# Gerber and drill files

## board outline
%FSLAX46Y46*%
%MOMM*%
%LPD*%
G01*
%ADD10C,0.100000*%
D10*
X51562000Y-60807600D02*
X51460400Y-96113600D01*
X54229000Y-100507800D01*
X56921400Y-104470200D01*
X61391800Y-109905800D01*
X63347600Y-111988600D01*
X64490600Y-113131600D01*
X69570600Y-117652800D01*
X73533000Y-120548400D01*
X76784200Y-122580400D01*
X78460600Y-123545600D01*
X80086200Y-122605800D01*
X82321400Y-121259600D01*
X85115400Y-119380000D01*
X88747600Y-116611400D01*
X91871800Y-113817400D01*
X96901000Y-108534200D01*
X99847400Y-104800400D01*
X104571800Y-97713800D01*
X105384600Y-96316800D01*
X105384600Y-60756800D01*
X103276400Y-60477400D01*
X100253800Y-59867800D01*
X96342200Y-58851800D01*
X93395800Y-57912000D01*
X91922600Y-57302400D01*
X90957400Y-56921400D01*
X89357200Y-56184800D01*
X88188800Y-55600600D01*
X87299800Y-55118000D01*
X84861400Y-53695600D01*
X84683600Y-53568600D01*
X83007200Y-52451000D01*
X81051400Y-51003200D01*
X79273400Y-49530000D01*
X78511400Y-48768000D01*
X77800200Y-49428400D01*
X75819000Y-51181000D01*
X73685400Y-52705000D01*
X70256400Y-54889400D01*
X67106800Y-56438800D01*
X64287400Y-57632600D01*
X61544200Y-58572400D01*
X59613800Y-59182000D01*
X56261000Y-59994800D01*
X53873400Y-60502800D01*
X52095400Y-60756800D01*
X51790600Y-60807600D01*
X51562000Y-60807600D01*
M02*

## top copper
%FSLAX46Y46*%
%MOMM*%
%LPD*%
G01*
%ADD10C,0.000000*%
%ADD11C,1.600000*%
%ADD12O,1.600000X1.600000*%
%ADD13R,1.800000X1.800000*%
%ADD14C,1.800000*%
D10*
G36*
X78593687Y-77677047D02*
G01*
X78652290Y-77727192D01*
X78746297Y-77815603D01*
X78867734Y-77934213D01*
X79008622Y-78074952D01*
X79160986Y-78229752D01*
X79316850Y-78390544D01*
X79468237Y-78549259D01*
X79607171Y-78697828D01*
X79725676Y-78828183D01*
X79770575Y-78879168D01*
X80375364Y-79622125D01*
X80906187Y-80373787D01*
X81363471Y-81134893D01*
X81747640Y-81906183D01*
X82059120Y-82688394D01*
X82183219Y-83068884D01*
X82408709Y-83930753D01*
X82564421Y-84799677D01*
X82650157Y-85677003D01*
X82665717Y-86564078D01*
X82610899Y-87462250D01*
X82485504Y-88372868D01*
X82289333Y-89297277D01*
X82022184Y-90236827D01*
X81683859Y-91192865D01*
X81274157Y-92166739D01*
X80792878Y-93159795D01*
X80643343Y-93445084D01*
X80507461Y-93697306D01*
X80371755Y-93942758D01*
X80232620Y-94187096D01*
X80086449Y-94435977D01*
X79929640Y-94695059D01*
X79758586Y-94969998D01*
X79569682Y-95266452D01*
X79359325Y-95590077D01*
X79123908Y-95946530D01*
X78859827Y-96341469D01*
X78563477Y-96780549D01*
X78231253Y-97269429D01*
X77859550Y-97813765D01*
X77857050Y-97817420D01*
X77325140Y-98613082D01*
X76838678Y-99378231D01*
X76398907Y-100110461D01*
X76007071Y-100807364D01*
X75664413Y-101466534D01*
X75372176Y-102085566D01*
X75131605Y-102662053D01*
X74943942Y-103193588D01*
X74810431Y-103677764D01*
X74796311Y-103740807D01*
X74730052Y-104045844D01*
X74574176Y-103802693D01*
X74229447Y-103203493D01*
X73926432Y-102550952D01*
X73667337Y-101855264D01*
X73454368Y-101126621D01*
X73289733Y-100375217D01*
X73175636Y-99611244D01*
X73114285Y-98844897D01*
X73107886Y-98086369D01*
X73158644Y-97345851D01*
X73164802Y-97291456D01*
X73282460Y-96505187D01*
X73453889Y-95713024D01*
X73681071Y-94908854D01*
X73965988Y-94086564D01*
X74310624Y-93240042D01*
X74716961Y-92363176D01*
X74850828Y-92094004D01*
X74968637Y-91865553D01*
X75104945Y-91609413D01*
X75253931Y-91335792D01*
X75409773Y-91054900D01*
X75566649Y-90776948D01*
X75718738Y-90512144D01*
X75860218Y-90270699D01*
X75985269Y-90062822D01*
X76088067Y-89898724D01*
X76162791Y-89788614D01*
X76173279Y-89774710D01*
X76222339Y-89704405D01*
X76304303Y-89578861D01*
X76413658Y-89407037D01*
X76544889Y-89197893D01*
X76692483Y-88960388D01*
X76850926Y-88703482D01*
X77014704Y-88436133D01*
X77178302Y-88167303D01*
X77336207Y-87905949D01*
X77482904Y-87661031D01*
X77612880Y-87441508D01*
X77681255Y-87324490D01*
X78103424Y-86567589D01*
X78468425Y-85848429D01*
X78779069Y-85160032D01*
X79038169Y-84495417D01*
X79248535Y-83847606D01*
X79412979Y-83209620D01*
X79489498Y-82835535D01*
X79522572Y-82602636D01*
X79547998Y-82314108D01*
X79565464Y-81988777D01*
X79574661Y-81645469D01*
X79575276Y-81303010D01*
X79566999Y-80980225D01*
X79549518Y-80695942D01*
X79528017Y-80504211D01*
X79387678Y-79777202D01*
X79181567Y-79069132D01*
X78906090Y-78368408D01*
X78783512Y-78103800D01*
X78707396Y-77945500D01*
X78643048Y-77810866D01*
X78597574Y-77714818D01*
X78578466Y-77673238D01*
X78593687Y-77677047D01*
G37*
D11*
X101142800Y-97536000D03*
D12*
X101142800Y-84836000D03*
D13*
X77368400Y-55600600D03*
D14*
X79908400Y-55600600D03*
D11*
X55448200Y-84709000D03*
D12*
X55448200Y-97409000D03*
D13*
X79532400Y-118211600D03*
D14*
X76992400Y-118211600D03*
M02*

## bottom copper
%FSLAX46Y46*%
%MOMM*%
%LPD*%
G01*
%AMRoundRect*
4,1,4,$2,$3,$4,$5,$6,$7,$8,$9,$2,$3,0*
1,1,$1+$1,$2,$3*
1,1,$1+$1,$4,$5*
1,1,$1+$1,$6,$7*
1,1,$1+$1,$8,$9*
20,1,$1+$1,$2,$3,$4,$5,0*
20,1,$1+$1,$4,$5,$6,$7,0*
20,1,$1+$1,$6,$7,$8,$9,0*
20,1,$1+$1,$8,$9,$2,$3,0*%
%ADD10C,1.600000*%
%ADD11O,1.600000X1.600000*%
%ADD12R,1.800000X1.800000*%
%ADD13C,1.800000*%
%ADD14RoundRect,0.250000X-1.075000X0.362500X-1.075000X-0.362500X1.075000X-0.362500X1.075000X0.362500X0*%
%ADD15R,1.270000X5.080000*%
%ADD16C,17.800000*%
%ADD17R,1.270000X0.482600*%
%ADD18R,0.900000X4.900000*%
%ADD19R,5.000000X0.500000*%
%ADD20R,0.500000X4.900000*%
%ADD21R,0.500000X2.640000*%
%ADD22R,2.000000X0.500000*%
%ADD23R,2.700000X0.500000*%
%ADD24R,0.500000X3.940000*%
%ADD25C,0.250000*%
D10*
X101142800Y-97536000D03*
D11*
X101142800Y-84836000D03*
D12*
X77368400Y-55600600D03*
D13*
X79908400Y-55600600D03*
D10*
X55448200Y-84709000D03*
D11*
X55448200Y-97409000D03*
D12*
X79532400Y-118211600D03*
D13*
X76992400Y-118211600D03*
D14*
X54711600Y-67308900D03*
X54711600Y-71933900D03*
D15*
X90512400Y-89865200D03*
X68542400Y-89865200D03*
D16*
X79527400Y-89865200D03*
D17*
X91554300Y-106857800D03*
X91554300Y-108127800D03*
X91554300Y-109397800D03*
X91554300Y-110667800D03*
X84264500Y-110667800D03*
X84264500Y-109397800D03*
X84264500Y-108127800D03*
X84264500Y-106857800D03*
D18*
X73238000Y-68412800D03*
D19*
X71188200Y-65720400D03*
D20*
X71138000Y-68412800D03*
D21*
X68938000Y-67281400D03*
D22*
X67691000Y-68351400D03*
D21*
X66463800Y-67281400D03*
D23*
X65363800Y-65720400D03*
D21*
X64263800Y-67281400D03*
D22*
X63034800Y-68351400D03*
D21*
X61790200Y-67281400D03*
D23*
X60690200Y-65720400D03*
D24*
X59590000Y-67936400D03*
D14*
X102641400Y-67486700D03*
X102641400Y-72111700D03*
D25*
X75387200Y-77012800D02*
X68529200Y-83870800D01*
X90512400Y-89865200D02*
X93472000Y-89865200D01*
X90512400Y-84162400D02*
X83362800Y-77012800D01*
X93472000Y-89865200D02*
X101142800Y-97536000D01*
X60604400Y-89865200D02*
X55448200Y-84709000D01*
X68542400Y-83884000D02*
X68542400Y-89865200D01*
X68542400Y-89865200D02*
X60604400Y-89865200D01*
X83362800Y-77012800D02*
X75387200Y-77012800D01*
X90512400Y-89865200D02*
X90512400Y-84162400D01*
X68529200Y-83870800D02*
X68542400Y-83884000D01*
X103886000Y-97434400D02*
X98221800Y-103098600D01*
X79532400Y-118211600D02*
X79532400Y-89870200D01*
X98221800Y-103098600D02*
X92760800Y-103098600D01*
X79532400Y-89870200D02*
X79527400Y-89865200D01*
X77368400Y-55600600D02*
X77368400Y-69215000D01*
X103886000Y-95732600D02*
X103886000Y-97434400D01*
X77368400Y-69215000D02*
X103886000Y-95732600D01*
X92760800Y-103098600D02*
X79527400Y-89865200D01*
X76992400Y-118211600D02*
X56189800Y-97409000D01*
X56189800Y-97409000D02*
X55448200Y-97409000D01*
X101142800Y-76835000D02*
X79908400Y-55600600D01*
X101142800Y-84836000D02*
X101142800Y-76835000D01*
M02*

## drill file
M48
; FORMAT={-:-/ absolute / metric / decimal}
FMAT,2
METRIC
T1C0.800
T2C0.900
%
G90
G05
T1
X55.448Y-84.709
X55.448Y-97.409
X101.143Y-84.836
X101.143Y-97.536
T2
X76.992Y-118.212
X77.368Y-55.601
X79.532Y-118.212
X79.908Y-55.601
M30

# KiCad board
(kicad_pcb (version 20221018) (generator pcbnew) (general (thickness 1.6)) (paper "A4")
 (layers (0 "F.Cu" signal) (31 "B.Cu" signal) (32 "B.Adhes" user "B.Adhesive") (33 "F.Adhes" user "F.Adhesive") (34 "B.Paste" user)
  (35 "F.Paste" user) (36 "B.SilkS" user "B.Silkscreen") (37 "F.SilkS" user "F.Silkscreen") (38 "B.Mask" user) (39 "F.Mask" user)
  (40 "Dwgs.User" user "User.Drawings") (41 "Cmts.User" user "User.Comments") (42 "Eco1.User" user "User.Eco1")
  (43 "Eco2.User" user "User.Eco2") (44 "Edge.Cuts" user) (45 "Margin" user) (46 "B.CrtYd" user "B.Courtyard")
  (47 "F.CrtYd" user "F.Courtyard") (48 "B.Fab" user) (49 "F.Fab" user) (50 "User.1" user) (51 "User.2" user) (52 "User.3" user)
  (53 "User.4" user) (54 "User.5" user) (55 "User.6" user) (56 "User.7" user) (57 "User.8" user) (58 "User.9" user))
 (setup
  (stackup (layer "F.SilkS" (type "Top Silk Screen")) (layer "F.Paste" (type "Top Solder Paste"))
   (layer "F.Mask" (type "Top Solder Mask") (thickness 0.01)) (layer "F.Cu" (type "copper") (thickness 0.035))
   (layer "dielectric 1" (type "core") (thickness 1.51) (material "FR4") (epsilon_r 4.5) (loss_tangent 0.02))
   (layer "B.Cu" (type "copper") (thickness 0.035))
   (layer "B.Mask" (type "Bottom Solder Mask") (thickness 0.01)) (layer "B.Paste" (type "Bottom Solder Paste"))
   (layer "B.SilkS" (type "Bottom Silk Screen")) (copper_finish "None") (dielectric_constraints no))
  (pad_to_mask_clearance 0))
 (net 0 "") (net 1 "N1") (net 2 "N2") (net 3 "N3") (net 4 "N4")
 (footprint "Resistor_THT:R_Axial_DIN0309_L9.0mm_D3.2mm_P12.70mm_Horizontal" (layer "F.Cu") (at 101.1428 97.536 90)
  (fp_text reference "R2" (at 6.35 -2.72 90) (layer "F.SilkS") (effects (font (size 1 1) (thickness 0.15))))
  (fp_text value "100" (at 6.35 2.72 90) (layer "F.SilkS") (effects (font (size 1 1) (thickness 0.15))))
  (pad "1" thru_hole circle (at 0 0 90) (size 1.6 1.6) (drill 0.8) (layers "*.Cu" "*.Mask") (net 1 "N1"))
  (pad "2" thru_hole oval (at 12.7 0 90) (size 1.6 1.6) (drill 0.8) (layers "*.Cu" "*.Mask") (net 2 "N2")))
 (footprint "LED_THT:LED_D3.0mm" (layer "F.Cu") (at 77.3684 55.6006)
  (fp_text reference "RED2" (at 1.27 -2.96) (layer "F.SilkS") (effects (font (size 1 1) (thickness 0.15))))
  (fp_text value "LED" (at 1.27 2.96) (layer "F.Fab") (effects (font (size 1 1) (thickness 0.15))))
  (pad "1" thru_hole rect (at 0 0) (size 1.8 1.8) (drill 0.9) (layers "*.Cu" "*.Mask") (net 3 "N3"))
  (pad "2" thru_hole circle (at 2.54 0) (size 1.8 1.8) (drill 0.9) (layers "*.Cu" "*.Mask") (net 2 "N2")))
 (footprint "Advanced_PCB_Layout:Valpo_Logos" (layer "F.Cu") (at 78.3844 88.3158)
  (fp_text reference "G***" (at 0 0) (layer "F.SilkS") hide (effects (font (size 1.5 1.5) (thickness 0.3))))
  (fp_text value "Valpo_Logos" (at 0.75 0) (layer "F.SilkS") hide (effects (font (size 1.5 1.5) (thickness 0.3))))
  (fp_poly
   (pts (xy 0.209287 -10.638753) (xy 0.26789 -10.588608) (xy 0.361897 -10.500197) (xy 0.483334 -10.381587) (xy 0.624222 -10.240848)
    (xy 0.776586 -10.086048) (xy 0.93245 -9.925256) (xy 1.083837 -9.766541) (xy 1.222771 -9.617972) (xy 1.341276 -9.487617)
    (xy 1.386175 -9.436632) (xy 1.990964 -8.693675) (xy 2.521787 -7.942013) (xy 2.979071 -7.180907) (xy 3.36324 -6.409617)
    (xy 3.67472 -5.627406) (xy 3.798819 -5.246916) (xy 4.024309 -4.385047) (xy 4.180021 -3.516123) (xy 4.265757 -2.638797)
    (xy 4.281317 -1.751722) (xy 4.226499 -0.85355) (xy 4.101104 0.057068) (xy 3.904933 0.981477) (xy 3.637784 1.921027)
    (xy 3.299459 2.877065) (xy 2.889757 3.850939) (xy 2.408478 4.843995) (xy 2.258943 5.129284) (xy 2.123061 5.381506)
    (xy 1.987355 5.626958) (xy 1.84822 5.871296) (xy 1.702049 6.120177) (xy 1.54524 6.379259) (xy 1.374186 6.654198) (xy 1.185282 6.950652)
    (xy 0.974925 7.274277) (xy 0.739508 7.63073) (xy 0.475427 8.025669) (xy 0.179077 8.464749) (xy -0.153147 8.953629)
    (xy -0.52485 9.497965) (xy -0.52735 9.50162) (xy -1.05926 10.297282) (xy -1.545722 11.062431) (xy -1.985493 11.794661)
    (xy -2.377329 12.491564) (xy -2.719987 13.150734) (xy -3.012224 13.769766) (xy -3.252795 14.346253) (xy -3.440458 14.877788)
    (xy -3.573969 15.361964) (xy -3.588089 15.425007) (xy -3.654348 15.730044) (xy -3.810224 15.486893) (xy -4.154953 14.887693)
    (xy -4.457968 14.235152) (xy -4.717063 13.539464) (xy -4.930032 12.810821) (xy -5.094667 12.059417) (xy -5.208764 11.295444)
    (xy -5.270115 10.529097) (xy -5.276514 9.770569) (xy -5.225756 9.030051) (xy -5.219598 8.975656) (xy -5.10194 8.189387)
    (xy -4.930511 7.397224) (xy -4.703329 6.593054) (xy -4.418412 5.770764) (xy -4.073776 4.924242) (xy -3.667439 4.047376)
    (xy -3.533572 3.778204) (xy -3.415763 3.549753) (xy -3.279455 3.293613) (xy -3.130469 3.019992) (xy -2.974627 2.7391)
    (xy -2.817751 2.461148) (xy -2.665662 2.196344) (xy -2.524182 1.954899) (xy -2.399131 1.747022) (xy -2.296333 1.582924)
    (xy -2.221609 1.472814) (xy -2.211121 1.45891) (xy -2.162061 1.388605) (xy -2.080097 1.263061) (xy -1.970742 1.091237)
    (xy -1.839511 0.882093) (xy -1.691917 0.644588) (xy -1.533474 0.387682) (xy -1.369696 0.120333) (xy -1.206098 -0.148497)
    (xy -1.048193 -0.409851) (xy -0.901496 -0.654769) (xy -0.77152 -0.874292) (xy -0.703145 -0.99131) (xy -0.280976 -1.748211)
    (xy 0.084025 -2.467371) (xy 0.394669 -3.155768) (xy 0.653769 -3.820383) (xy 0.864135 -4.468194) (xy 1.028579 -5.10618)
    (xy 1.105098 -5.480265) (xy 1.138172 -5.713164) (xy 1.163598 -6.001692) (xy 1.181064 -6.327023) (xy 1.190261 -6.670331)
    (xy 1.190876 -7.01279) (xy 1.182599 -7.335575) (xy 1.165118 -7.619858) (xy 1.143617 -7.811589) (xy 1.003278 -8.538598)
    (xy 0.797167 -9.246668) (xy 0.52169 -9.947392) (xy 0.399112 -10.212) (xy 0.322996 -10.3703) (xy 0.258648 -10.504934)
    (xy 0.213174 -10.600982) (xy 0.194066 -10.642562))
   (stroke (width 0) (type solid)) (fill solid) (layer "F.Cu")))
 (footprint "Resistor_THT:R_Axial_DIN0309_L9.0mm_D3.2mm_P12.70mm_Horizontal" (layer "F.Cu") (at 55.4482 84.709 -90)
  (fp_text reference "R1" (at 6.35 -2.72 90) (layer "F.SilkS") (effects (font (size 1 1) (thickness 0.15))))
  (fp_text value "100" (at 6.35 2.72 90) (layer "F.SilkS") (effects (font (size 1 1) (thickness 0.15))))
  (pad "1" thru_hole circle (at 0 0 270) (size 1.6 1.6) (drill 0.8) (layers "*.Cu" "*.Mask") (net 1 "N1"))
  (pad "2" thru_hole oval (at 12.7 0 270) (size 1.6 1.6) (drill 0.8) (layers "*.Cu" "*.Mask") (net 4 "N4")))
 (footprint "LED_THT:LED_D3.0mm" (layer "F.Cu") (at 79.5324 118.2116 180)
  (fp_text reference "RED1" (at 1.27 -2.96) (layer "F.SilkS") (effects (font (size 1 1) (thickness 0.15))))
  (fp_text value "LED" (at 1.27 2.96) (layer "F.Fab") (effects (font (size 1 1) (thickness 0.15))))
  (pad "1" thru_hole rect (at 0 0 180) (size 1.8 1.8) (drill 0.9) (layers "*.Cu" "*.Mask") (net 3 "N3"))
  (pad "2" thru_hole circle (at 2.54 0 180) (size 1.8 1.8) (drill 0.9) (layers "*.Cu" "*.Mask") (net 4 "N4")))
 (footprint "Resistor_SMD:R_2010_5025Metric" (layer "B.Cu") (at 54.7116 69.6214 -90)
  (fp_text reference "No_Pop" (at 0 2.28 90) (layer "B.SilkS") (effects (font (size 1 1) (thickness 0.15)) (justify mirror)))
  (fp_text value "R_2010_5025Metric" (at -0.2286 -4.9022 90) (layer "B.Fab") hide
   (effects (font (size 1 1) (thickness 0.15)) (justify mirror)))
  (pad "1" smd roundrect (at -2.3125 0 270) (size 1.225 2.65) (layers "B.Cu" "B.Paste" "B.Mask") (roundrect_rratio 0.204082))
  (pad "2" smd roundrect (at 2.3125 0 270) (size 1.225 2.65) (layers "B.Cu" "B.Paste" "B.Mask") (roundrect_rratio 0.204082)))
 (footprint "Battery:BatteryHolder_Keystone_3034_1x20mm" (layer "B.Cu") (at 79.5274 89.8652 180)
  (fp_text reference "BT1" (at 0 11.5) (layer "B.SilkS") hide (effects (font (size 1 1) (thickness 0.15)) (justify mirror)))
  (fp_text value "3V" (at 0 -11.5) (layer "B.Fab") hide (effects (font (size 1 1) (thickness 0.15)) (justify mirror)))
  (pad "1" smd rect (at -10.985 0 180) (size 1.27 5.08) (layers "B.Cu" "B.Paste" "B.Mask") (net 1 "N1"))
  (pad "1" smd rect (at 10.985 0 180) (size 1.27 5.08) (layers "B.Cu" "B.Paste" "B.Mask") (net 1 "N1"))
  (pad "2" smd circle (at 0 0 180) (size 17.8 17.8) (layers "B.Cu" "B.Mask") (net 3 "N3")))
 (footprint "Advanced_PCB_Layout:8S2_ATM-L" (layer "B.Cu") (at 87.9094 108.7628 180)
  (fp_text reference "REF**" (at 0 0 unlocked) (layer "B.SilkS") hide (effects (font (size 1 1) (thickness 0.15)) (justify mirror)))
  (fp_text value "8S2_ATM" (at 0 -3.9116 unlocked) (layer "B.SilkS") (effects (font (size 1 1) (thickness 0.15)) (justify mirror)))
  (pad "1" smd rect (at -3.6449 1.905 180) (size 1.27 0.4826) (layers "B.Cu" "B.Paste" "B.Mask"))
  (pad "2" smd rect (at -3.6449 0.635 180) (size 1.27 0.4826) (layers "B.Cu" "B.Paste" "B.Mask"))
  (pad "3" smd rect (at -3.6449 -0.635 180) (size 1.27 0.4826) (layers "B.Cu" "B.Paste" "B.Mask"))
  (pad "4" smd rect (at -3.6449 -1.905 180) (size 1.27 0.4826) (layers "B.Cu" "B.Paste" "B.Mask"))
  (pad "5" smd rect (at 3.6449 -1.905 180) (size 1.27 0.4826) (layers "B.Cu" "B.Paste" "B.Mask"))
  (pad "6" smd rect (at 3.6449 -0.635 180) (size 1.27 0.4826) (layers "B.Cu" "B.Paste" "B.Mask"))
  (pad "7" smd rect (at 3.6449 0.635 180) (size 1.27 0.4826) (layers "B.Cu" "B.Paste" "B.Mask"))
  (pad "8" smd rect (at 3.6449 1.905 180) (size 1.27 0.4826) (layers "B.Cu" "B.Paste" "B.Mask")))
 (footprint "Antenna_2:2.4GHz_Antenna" (layer "B.Cu") (at 66.921 73.7214 180)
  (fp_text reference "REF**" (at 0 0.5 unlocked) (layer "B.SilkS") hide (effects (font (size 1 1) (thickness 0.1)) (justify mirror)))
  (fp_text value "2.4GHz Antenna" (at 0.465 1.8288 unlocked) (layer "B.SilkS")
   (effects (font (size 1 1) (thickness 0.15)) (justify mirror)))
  (pad "1" smd rect (at -6.317 5.3086 90) (size 4.9 0.9) (layers "B.Cu" "B.Paste" "B.Mask") (thermal_bridge_angle 45))
  (pad "1" smd rect (at -4.2672 8.001 180) (size 5 0.5) (layers "B.Cu" "B.Paste" "B.Mask") (thermal_bridge_angle 45))
  (pad "1" smd rect (at -4.217 5.3086 90) (size 4.9 0.5) (layers "B.Cu" "B.Paste" "B.Mask") (thermal_bridge_angle 45))
  (pad "1" smd rect (at -2.017 6.44 90) (size 2.64 0.5) (layers "B.Cu" "B.Paste" "B.Mask") (thermal_bridge_angle 45))
  (pad "1" smd rect (at -0.77 5.37 180) (size 2 0.5) (layers "B.Cu" "B.Paste" "B.Mask") (thermal_bridge_angle 45))
  (pad "1" smd rect (at 0.4572 6.44 90) (size 2.64 0.5) (layers "B.Cu" "B.Paste" "B.Mask") (thermal_bridge_angle 45))
  (pad "1" smd rect (at 1.5572 8.001 180) (size 2.7 0.5) (layers "B.Cu" "B.Paste" "B.Mask") (thermal_bridge_angle 45))
  (pad "1" smd rect (at 2.6572 6.44 90) (size 2.64 0.5) (layers "B.Cu" "B.Paste" "B.Mask") (thermal_bridge_angle 45))
  (pad "1" smd rect (at 3.8862 5.37 180) (size 2 0.5) (layers "B.Cu" "B.Paste" "B.Mask") (thermal_bridge_angle 45))
  (pad "1" smd rect (at 5.1308 6.44 90) (size 2.64 0.5) (layers "B.Cu" "B.Paste" "B.Mask") (thermal_bridge_angle 45))
  (pad "1" smd rect (at 6.2308 8.001 180) (size 2.7 0.5) (layers "B.Cu" "B.Paste" "B.Mask") (thermal_bridge_angle 45))
  (pad "1" smd rect (at 7.331 5.785 90) (size 3.94 0.5) (layers "B.Cu" "B.Paste" "B.Mask") (thermal_bridge_angle 45)))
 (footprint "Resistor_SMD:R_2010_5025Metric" (layer "B.Cu") (at 102.6414 69.7992 -90)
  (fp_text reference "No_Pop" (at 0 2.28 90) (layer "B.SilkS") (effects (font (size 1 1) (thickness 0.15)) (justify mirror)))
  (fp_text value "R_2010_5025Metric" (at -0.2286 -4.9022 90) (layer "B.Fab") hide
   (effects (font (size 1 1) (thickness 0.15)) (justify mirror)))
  (pad "1" smd roundrect (at -2.3125 0 270) (size 1.225 2.65) (layers "B.Cu" "B.Paste" "B.Mask") (roundrect_rratio 0.204082))
  (pad "2" smd roundrect (at 2.3125 0 270) (size 1.225 2.65) (layers "B.Cu" "B.Paste" "B.Mask") (roundrect_rratio 0.204082)))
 (gr_poly
  (pts (xy 51.562 60.8076) (xy 51.4604 96.1136) (xy 54.229 100.5078) (xy 56.9214 104.4702) (xy 61.3918 109.9058) (xy 63.3476 111.9886)
   (xy 64.4906 113.1316) (xy 69.5706 117.6528) (xy 73.533 120.5484) (xy 76.7842 122.5804) (xy 78.4606 123.5456) (xy 80.0862 122.6058)
   (xy 82.3214 121.2596) (xy 85.1154 119.38) (xy 88.7476 116.6114) (xy 91.8718 113.8174) (xy 96.901 108.5342) (xy 99.8474 104.8004)
   (xy 104.5718 97.7138) (xy 105.3846 96.3168) (xy 105.3846 60.7568) (xy 103.2764 60.4774) (xy 100.2538 59.8678) (xy 96.3422 58.8518)
   (xy 93.3958 57.912) (xy 91.9226 57.3024) (xy 90.9574 56.9214) (xy 89.3572 56.1848) (xy 88.1888 55.6006) (xy 87.2998 55.118)
   (xy 84.8614 53.6956) (xy 84.6836 53.5686) (xy 83.0072 52.451) (xy 81.0514 51.0032) (xy 79.2734 49.53) (xy 78.5114 48.768)
   (xy 77.8002 49.4284) (xy 75.819 51.181) (xy 73.6854 52.705) (xy 70.2564 54.8894) (xy 67.1068 56.4388) (xy 64.2874 57.6326)
   (xy 61.5442 58.5724) (xy 59.6138 59.182) (xy 56.261 59.9948) (xy 53.8734 60.5028) (xy 52.0954 60.7568) (xy 51.7906 60.8076))
  (stroke (width 0.1) (type solid)) (fill none) (layer "Edge.Cuts"))
 (segment (start 75.3872 77.0128) (end 68.5292 83.8708) (width 0.25) (layer "B.Cu") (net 1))
 (segment (start 90.5124 89.8652) (end 93.472 89.8652) (width 0.25) (layer "B.Cu") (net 1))
 (segment (start 90.5124 84.1624) (end 83.3628 77.0128) (width 0.25) (layer "B.Cu") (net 1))
 (segment (start 93.472 89.8652) (end 101.1428 97.536) (width 0.25) (layer "B.Cu") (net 1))
 (segment (start 60.6044 89.8652) (end 55.4482 84.709) (width 0.25) (layer "B.Cu") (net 1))
 (segment (start 68.5424 83.884) (end 68.5424 89.8652) (width 0.25) (layer "B.Cu") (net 1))
 (segment (start 68.5424 89.8652) (end 60.6044 89.8652) (width 0.25) (layer "B.Cu") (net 1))
 (segment (start 83.3628 77.0128) (end 75.3872 77.0128) (width 0.25) (layer "B.Cu") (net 1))
 (segment (start 90.5124 89.8652) (end 90.5124 84.1624) (width 0.25) (layer "B.Cu") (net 1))
 (segment (start 68.5292 83.8708) (end 68.5424 83.884) (width 0.25) (layer "B.Cu") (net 1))
 (segment (start 103.886 97.4344) (end 98.2218 103.0986) (width 0.25) (layer "B.Cu") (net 3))
 (segment (start 79.5324 118.2116) (end 79.5324 89.8702) (width 0.25) (layer "B.Cu") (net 3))
 (segment (start 98.2218 103.0986) (end 92.7608 103.0986) (width 0.25) (layer "B.Cu") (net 3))
 (segment (start 79.5324 89.8702) (end 79.5274 89.8652) (width 0.25) (layer "B.Cu") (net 3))
 (segment (start 77.3684 55.6006) (end 77.3684 69.215) (width 0.25) (layer "B.Cu") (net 3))
 (segment (start 103.886 95.7326) (end 103.886 97.4344) (width 0.25) (layer "B.Cu") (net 3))
 (segment (start 77.3684 69.215) (end 103.886 95.7326) (width 0.25) (layer "B.Cu") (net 3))
 (segment (start 92.7608 103.0986) (end 79.5274 89.8652) (width 0.25) (layer "B.Cu") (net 3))
 (segment (start 76.9924 118.2116) (end 56.1898 97.409) (width 0.25) (layer "B.Cu") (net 4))
 (segment (start 56.1898 97.409) (end 55.4482 97.409) (width 0.25) (layer "B.Cu") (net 4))
 (segment (start 101.1428 76.835) (end 79.9084 55.6006) (width 0.25) (layer "B.Cu") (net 2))
 (segment (start 101.1428 84.836) (end 101.1428 76.835) (width 0.25) (layer "B.Cu") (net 2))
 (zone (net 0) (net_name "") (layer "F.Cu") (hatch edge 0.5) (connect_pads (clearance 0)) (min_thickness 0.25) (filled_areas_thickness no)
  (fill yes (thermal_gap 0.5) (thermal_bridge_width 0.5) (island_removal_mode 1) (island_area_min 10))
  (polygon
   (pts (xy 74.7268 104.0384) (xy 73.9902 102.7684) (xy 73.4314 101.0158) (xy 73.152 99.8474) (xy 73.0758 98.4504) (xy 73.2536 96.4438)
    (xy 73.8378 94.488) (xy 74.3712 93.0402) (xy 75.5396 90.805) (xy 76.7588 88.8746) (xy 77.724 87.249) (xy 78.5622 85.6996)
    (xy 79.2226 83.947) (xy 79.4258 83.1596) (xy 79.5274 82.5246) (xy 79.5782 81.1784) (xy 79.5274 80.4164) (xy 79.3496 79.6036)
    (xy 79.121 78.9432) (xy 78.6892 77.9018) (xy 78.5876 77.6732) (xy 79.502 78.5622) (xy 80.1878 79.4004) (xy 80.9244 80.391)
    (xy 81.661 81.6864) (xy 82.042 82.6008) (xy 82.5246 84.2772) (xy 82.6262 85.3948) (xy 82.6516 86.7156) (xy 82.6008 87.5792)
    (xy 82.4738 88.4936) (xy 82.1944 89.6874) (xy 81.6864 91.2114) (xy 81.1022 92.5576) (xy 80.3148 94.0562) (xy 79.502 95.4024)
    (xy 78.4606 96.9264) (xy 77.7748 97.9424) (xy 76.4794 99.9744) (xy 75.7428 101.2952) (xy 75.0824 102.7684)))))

